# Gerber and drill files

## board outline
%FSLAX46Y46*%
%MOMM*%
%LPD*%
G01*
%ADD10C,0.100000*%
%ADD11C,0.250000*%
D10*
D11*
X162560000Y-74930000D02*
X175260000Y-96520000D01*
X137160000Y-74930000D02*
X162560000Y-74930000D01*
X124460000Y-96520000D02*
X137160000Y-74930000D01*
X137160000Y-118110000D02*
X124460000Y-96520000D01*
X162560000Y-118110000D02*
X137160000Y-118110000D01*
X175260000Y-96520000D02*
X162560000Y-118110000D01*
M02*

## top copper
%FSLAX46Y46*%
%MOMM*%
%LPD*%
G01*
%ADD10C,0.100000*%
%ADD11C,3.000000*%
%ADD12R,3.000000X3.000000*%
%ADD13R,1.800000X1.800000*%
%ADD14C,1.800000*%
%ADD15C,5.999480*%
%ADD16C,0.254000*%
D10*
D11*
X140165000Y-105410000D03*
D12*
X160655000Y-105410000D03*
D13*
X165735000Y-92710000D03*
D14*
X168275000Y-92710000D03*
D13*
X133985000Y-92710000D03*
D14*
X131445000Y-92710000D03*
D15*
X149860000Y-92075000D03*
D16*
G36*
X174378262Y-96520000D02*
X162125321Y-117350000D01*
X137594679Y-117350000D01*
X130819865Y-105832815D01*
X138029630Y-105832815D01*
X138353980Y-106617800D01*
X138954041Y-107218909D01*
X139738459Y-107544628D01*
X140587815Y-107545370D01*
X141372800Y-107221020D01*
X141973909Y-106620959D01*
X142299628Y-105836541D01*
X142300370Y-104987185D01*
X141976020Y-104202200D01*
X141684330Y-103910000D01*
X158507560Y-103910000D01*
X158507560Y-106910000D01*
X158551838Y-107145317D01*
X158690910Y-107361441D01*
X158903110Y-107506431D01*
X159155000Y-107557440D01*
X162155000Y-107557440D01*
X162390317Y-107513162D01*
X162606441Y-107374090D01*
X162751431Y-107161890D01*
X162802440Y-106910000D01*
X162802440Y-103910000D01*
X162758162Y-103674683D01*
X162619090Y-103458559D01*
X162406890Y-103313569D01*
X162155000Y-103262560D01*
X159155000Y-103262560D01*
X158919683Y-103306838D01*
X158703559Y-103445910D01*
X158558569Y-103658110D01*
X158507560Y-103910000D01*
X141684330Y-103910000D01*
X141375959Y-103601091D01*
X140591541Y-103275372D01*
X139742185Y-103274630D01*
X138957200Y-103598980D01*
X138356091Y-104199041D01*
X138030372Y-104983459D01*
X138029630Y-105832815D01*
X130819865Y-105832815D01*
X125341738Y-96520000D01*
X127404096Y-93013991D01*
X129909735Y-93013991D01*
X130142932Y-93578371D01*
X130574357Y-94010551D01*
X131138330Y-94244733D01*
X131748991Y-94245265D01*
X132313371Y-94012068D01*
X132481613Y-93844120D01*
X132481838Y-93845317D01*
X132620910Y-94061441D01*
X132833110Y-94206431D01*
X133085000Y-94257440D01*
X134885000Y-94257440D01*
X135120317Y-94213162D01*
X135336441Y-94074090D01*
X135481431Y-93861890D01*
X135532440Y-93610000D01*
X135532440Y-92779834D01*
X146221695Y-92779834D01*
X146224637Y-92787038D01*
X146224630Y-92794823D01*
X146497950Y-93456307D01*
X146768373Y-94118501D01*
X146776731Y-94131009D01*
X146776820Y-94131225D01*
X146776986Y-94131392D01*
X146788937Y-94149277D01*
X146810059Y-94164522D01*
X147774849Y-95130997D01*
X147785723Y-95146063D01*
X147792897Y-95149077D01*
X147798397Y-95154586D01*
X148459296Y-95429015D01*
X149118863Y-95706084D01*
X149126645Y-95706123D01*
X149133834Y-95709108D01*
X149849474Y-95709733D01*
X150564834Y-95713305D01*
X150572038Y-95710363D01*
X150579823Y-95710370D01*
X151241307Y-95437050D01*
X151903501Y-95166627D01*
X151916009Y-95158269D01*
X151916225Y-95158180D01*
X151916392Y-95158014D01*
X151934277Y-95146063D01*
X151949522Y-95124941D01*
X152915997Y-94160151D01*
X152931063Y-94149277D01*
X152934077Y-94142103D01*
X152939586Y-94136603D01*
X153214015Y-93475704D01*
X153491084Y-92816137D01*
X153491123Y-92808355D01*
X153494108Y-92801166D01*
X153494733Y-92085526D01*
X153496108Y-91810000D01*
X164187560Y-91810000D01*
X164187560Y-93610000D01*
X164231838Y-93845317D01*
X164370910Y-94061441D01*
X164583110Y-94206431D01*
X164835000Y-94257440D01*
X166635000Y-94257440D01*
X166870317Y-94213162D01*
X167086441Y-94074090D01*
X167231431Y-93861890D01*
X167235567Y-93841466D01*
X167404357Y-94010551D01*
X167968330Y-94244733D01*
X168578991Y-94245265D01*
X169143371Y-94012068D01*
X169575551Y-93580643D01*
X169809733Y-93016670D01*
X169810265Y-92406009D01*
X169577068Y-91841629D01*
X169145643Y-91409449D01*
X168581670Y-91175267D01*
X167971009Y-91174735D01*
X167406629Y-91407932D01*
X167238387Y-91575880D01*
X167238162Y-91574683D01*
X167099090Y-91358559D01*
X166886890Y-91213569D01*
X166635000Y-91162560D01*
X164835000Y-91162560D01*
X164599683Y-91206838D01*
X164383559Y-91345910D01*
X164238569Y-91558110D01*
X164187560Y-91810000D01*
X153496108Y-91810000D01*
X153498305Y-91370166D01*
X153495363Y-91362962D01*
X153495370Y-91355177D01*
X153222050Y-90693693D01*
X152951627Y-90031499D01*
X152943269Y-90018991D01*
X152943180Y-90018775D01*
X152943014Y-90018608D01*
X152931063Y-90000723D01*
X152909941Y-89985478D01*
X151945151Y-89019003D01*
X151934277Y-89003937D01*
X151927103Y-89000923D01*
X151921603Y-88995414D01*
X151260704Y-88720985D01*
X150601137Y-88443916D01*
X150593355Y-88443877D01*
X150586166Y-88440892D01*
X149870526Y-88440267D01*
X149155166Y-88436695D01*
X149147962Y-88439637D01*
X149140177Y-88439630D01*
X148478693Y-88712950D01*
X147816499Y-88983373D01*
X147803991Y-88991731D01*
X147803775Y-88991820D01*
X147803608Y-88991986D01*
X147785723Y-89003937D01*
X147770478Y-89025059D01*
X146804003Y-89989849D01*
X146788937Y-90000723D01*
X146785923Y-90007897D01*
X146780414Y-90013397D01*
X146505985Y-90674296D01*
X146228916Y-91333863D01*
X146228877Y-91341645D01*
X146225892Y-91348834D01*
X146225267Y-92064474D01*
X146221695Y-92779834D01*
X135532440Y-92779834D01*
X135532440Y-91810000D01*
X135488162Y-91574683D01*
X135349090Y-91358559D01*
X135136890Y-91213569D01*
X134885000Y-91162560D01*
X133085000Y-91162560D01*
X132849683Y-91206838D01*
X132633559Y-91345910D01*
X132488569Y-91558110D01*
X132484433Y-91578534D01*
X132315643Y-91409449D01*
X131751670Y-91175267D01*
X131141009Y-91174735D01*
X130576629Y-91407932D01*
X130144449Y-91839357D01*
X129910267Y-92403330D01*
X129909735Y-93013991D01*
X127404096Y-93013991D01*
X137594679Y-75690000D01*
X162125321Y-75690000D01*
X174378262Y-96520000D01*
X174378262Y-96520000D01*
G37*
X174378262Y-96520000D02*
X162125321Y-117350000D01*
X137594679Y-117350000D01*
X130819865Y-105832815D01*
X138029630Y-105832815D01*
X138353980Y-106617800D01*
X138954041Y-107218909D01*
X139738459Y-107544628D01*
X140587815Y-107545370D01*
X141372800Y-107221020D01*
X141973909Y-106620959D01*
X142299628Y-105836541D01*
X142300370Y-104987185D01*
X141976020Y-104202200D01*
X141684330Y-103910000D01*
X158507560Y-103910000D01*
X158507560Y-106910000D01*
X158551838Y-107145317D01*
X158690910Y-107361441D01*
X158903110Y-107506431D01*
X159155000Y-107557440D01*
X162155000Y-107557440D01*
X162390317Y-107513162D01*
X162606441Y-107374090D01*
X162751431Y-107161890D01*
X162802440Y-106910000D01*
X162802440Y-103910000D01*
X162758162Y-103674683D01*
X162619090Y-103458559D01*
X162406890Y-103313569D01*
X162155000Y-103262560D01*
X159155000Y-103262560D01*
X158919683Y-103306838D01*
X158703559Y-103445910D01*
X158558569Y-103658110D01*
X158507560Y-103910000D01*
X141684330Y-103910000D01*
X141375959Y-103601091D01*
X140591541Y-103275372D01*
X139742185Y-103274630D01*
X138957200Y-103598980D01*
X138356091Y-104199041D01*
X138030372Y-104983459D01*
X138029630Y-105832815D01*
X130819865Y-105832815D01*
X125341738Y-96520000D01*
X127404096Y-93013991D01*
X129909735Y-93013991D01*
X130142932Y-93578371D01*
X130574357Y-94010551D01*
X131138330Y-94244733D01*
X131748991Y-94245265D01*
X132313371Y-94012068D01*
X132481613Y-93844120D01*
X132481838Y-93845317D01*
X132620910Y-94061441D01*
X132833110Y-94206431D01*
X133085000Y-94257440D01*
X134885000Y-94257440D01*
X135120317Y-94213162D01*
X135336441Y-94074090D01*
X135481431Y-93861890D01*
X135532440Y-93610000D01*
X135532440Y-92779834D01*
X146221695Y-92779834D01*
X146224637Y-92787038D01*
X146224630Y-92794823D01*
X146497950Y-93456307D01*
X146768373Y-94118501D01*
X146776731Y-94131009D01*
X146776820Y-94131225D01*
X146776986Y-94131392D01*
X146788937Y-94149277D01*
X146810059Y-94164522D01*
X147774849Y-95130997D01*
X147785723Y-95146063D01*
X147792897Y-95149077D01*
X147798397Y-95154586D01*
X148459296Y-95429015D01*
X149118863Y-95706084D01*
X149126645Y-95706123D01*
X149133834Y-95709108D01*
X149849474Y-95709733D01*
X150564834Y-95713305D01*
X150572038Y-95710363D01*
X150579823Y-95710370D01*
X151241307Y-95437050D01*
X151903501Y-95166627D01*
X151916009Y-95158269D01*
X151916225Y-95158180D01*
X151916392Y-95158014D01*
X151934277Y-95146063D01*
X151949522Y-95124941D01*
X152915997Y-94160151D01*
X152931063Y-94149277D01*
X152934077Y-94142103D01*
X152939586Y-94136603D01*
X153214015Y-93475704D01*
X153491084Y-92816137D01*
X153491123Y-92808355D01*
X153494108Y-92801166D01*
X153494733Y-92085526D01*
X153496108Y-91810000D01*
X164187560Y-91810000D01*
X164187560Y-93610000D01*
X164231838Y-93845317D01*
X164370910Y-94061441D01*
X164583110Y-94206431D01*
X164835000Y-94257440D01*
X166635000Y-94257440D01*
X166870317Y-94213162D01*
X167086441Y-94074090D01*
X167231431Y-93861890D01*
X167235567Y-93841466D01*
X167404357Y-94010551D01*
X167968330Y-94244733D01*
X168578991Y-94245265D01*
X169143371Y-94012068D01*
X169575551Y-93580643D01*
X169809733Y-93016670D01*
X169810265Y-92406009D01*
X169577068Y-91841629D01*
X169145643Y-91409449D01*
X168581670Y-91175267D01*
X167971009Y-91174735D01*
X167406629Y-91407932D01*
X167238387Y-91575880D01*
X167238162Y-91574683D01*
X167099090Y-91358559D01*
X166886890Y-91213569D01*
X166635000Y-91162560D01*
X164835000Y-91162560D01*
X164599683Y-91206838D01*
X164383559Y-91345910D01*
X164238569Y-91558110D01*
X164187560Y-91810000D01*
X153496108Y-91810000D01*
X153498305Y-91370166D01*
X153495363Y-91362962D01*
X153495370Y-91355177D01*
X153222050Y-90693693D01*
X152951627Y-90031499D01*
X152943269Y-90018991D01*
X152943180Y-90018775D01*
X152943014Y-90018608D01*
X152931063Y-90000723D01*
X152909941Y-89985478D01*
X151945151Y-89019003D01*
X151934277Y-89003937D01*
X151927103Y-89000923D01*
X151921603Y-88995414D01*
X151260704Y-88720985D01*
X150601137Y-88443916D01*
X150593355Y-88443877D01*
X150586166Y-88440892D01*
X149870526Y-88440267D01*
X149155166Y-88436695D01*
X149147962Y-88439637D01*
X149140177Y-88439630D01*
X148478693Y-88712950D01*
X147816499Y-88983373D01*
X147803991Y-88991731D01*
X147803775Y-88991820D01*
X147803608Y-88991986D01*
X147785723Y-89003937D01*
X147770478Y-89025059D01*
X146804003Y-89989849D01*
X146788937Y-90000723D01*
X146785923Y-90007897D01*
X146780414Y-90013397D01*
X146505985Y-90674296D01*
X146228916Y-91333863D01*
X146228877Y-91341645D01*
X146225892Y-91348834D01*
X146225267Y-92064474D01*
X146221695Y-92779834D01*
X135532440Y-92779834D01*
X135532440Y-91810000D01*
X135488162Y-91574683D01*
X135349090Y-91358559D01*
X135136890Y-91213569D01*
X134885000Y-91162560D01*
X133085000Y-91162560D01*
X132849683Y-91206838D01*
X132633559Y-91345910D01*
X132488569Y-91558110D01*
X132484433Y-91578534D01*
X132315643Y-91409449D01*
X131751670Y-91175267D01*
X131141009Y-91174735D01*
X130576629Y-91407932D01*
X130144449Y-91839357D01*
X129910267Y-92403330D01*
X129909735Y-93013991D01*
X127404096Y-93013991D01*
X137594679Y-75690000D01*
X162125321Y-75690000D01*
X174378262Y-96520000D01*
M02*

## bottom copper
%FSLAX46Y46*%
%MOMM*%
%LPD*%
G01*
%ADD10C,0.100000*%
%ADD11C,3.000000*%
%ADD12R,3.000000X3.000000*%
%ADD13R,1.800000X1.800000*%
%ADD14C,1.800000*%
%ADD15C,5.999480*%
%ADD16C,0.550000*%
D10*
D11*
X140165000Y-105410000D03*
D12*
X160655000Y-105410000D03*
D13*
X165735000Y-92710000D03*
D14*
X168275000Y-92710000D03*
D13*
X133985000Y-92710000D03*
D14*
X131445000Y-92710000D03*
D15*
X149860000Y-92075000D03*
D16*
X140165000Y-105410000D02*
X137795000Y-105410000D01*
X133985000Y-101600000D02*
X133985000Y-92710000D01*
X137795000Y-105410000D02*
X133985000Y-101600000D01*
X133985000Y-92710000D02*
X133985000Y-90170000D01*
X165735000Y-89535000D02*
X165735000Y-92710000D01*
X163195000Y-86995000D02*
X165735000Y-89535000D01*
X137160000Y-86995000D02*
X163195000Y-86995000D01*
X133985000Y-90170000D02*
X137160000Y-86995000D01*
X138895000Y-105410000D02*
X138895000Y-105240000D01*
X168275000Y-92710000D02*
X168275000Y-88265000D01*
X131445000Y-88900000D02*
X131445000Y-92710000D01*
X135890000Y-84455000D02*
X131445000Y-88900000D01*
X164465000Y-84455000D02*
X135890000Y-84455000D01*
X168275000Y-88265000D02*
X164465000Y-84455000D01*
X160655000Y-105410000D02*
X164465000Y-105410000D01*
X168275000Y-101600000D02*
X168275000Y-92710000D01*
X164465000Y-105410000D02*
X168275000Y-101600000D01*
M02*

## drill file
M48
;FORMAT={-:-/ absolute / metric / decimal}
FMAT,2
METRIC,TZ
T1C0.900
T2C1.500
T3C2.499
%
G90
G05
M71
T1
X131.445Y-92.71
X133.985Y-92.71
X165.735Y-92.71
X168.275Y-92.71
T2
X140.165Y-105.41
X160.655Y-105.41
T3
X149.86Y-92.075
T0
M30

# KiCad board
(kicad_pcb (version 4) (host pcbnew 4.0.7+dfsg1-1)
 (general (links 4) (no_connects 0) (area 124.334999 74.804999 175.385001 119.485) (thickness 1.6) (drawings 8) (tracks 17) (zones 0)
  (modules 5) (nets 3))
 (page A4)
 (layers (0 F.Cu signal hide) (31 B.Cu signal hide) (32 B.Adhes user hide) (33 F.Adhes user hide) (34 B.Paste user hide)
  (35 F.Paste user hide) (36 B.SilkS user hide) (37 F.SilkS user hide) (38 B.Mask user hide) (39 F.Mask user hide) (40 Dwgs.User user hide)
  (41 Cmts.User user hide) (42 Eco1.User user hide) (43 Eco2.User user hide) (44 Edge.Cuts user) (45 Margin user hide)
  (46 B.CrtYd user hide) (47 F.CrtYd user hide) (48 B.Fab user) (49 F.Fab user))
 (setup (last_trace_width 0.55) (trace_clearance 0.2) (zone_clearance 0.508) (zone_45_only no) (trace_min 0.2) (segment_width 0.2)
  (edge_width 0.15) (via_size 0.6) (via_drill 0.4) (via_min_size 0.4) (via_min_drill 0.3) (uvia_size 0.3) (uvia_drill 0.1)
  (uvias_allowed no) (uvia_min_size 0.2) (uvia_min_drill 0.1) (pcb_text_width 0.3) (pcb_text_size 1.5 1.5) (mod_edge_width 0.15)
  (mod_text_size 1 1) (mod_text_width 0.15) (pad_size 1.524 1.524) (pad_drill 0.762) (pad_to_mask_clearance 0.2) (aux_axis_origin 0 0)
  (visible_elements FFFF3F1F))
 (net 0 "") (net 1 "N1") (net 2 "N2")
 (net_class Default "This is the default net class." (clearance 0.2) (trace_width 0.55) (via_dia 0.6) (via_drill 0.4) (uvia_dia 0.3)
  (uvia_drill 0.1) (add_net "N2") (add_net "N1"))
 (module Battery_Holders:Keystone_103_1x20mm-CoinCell (layer B.Cu) (at 160.655 105.41 180)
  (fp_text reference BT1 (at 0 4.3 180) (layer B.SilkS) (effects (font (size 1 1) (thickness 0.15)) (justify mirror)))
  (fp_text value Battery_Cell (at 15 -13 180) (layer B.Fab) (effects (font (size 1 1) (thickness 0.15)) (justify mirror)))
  (pad 2 thru_hole circle (at 20.49 0 180) (size 3 3) (drill 1.5) (layers *.Cu *.Mask) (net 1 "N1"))
  (pad 1 thru_hole rect (at 0 0 180) (size 3 3) (drill 1.5) (layers *.Cu *.Mask) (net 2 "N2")))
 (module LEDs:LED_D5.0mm (layer B.Cu) (at 165.735 92.71)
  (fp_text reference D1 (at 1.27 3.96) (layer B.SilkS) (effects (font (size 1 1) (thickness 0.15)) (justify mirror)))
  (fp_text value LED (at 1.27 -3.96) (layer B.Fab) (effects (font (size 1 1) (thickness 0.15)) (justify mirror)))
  (pad 1 thru_hole rect (at 0 0) (size 1.8 1.8) (drill 0.9) (layers *.Cu *.Mask) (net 1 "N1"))
  (pad 2 thru_hole circle (at 2.54 0) (size 1.8 1.8) (drill 0.9) (layers *.Cu *.Mask) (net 2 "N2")))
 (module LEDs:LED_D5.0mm (layer B.Cu) (at 133.985 92.71 180)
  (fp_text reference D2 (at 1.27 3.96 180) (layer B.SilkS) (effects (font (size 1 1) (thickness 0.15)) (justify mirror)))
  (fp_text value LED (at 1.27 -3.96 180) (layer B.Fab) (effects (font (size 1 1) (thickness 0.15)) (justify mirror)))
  (pad 1 thru_hole rect (at 0 0 180) (size 1.8 1.8) (drill 0.9) (layers *.Cu *.Mask) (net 1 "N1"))
  (pad 2 thru_hole circle (at 2.54 0 180) (size 1.8 1.8) (drill 0.9) (layers *.Cu *.Mask) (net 2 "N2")))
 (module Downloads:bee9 (layer F.Cu) (at 150.495 94.615)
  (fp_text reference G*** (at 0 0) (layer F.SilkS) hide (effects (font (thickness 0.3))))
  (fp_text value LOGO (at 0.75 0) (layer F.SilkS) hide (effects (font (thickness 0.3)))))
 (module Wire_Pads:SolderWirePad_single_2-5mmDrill (layer F.Cu) (at 149.86 92.075)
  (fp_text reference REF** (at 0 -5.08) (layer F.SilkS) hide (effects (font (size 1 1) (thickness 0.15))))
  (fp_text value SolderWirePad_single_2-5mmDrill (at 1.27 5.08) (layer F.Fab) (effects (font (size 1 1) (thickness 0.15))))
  (pad 1 thru_hole circle (at 0 0) (size 5.99948 5.99948) (drill 2.49936) (layers *.Cu *.Mask)))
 (gr_line (start 162.56 74.93) (end 175.26 96.52) (angle 90) (layer Edge.Cuts) (width 0.25))
 (gr_line (start 137.16 74.93) (end 162.56 74.93) (angle 90) (layer Edge.Cuts) (width 0.25))
 (gr_line (start 124.46 96.52) (end 137.16 74.93) (angle 90) (layer Edge.Cuts) (width 0.25))
 (gr_line (start 137.16 118.11) (end 124.46 96.52) (angle 90) (layer Edge.Cuts) (width 0.25))
 (gr_line (start 162.56 118.11) (end 137.16 118.11) (angle 90) (layer Edge.Cuts) (width 0.25))
 (gr_line (start 175.26 96.52) (end 162.56 118.11) (angle 90) (layer Edge.Cuts) (width 0.25))
 (segment (start 140.165 105.41) (end 137.795 105.41) (width 0.55) (layer B.Cu) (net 1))
 (segment (start 133.985 101.6) (end 133.985 92.71) (width 0.55) (layer B.Cu) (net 1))
 (segment (start 137.795 105.41) (end 133.985 101.6) (width 0.55) (layer B.Cu) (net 1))
 (segment (start 133.985 92.71) (end 133.985 90.17) (width 0.55) (layer B.Cu) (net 1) (status 10))
 (segment (start 165.735 89.535) (end 165.735 92.71) (width 0.55) (layer B.Cu) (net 1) (status 20))
 (segment (start 163.195 86.995) (end 165.735 89.535) (width 0.55) (layer B.Cu) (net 1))
 (segment (start 137.16 86.995) (end 163.195 86.995) (width 0.55) (layer B.Cu) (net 1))
 (segment (start 133.985 90.17) (end 137.16 86.995) (width 0.55) (layer B.Cu) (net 1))
 (segment (start 138.895 105.41) (end 138.895 105.24) (width 0.55) (layer B.Cu) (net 1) (status 30))
 (segment (start 168.275 92.71) (end 168.275 88.265) (width 0.55) (layer B.Cu) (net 2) (status 10))
 (segment (start 131.445 88.9) (end 131.445 92.71) (width 0.55) (layer B.Cu) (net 2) (status 20))
 (segment (start 135.89 84.455) (end 131.445 88.9) (width 0.55) (layer B.Cu) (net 2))
 (segment (start 164.465 84.455) (end 135.89 84.455) (width 0.55) (layer B.Cu) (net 2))
 (segment (start 168.275 88.265) (end 164.465 84.455) (width 0.55) (layer B.Cu) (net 2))
 (segment (start 160.655 105.41) (end 164.465 105.41) (width 0.55) (layer B.Cu) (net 2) (status 10))
 (segment (start 168.275 101.6) (end 168.275 92.71) (width 0.55) (layer B.Cu) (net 2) (status 20))
 (segment (start 164.465 105.41) (end 168.275 101.6) (width 0.55) (layer B.Cu) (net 2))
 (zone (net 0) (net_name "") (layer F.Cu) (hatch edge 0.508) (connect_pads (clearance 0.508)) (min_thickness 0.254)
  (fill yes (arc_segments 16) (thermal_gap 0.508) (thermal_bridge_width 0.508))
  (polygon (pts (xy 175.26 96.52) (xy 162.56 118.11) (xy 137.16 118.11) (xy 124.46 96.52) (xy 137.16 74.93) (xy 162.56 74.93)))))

